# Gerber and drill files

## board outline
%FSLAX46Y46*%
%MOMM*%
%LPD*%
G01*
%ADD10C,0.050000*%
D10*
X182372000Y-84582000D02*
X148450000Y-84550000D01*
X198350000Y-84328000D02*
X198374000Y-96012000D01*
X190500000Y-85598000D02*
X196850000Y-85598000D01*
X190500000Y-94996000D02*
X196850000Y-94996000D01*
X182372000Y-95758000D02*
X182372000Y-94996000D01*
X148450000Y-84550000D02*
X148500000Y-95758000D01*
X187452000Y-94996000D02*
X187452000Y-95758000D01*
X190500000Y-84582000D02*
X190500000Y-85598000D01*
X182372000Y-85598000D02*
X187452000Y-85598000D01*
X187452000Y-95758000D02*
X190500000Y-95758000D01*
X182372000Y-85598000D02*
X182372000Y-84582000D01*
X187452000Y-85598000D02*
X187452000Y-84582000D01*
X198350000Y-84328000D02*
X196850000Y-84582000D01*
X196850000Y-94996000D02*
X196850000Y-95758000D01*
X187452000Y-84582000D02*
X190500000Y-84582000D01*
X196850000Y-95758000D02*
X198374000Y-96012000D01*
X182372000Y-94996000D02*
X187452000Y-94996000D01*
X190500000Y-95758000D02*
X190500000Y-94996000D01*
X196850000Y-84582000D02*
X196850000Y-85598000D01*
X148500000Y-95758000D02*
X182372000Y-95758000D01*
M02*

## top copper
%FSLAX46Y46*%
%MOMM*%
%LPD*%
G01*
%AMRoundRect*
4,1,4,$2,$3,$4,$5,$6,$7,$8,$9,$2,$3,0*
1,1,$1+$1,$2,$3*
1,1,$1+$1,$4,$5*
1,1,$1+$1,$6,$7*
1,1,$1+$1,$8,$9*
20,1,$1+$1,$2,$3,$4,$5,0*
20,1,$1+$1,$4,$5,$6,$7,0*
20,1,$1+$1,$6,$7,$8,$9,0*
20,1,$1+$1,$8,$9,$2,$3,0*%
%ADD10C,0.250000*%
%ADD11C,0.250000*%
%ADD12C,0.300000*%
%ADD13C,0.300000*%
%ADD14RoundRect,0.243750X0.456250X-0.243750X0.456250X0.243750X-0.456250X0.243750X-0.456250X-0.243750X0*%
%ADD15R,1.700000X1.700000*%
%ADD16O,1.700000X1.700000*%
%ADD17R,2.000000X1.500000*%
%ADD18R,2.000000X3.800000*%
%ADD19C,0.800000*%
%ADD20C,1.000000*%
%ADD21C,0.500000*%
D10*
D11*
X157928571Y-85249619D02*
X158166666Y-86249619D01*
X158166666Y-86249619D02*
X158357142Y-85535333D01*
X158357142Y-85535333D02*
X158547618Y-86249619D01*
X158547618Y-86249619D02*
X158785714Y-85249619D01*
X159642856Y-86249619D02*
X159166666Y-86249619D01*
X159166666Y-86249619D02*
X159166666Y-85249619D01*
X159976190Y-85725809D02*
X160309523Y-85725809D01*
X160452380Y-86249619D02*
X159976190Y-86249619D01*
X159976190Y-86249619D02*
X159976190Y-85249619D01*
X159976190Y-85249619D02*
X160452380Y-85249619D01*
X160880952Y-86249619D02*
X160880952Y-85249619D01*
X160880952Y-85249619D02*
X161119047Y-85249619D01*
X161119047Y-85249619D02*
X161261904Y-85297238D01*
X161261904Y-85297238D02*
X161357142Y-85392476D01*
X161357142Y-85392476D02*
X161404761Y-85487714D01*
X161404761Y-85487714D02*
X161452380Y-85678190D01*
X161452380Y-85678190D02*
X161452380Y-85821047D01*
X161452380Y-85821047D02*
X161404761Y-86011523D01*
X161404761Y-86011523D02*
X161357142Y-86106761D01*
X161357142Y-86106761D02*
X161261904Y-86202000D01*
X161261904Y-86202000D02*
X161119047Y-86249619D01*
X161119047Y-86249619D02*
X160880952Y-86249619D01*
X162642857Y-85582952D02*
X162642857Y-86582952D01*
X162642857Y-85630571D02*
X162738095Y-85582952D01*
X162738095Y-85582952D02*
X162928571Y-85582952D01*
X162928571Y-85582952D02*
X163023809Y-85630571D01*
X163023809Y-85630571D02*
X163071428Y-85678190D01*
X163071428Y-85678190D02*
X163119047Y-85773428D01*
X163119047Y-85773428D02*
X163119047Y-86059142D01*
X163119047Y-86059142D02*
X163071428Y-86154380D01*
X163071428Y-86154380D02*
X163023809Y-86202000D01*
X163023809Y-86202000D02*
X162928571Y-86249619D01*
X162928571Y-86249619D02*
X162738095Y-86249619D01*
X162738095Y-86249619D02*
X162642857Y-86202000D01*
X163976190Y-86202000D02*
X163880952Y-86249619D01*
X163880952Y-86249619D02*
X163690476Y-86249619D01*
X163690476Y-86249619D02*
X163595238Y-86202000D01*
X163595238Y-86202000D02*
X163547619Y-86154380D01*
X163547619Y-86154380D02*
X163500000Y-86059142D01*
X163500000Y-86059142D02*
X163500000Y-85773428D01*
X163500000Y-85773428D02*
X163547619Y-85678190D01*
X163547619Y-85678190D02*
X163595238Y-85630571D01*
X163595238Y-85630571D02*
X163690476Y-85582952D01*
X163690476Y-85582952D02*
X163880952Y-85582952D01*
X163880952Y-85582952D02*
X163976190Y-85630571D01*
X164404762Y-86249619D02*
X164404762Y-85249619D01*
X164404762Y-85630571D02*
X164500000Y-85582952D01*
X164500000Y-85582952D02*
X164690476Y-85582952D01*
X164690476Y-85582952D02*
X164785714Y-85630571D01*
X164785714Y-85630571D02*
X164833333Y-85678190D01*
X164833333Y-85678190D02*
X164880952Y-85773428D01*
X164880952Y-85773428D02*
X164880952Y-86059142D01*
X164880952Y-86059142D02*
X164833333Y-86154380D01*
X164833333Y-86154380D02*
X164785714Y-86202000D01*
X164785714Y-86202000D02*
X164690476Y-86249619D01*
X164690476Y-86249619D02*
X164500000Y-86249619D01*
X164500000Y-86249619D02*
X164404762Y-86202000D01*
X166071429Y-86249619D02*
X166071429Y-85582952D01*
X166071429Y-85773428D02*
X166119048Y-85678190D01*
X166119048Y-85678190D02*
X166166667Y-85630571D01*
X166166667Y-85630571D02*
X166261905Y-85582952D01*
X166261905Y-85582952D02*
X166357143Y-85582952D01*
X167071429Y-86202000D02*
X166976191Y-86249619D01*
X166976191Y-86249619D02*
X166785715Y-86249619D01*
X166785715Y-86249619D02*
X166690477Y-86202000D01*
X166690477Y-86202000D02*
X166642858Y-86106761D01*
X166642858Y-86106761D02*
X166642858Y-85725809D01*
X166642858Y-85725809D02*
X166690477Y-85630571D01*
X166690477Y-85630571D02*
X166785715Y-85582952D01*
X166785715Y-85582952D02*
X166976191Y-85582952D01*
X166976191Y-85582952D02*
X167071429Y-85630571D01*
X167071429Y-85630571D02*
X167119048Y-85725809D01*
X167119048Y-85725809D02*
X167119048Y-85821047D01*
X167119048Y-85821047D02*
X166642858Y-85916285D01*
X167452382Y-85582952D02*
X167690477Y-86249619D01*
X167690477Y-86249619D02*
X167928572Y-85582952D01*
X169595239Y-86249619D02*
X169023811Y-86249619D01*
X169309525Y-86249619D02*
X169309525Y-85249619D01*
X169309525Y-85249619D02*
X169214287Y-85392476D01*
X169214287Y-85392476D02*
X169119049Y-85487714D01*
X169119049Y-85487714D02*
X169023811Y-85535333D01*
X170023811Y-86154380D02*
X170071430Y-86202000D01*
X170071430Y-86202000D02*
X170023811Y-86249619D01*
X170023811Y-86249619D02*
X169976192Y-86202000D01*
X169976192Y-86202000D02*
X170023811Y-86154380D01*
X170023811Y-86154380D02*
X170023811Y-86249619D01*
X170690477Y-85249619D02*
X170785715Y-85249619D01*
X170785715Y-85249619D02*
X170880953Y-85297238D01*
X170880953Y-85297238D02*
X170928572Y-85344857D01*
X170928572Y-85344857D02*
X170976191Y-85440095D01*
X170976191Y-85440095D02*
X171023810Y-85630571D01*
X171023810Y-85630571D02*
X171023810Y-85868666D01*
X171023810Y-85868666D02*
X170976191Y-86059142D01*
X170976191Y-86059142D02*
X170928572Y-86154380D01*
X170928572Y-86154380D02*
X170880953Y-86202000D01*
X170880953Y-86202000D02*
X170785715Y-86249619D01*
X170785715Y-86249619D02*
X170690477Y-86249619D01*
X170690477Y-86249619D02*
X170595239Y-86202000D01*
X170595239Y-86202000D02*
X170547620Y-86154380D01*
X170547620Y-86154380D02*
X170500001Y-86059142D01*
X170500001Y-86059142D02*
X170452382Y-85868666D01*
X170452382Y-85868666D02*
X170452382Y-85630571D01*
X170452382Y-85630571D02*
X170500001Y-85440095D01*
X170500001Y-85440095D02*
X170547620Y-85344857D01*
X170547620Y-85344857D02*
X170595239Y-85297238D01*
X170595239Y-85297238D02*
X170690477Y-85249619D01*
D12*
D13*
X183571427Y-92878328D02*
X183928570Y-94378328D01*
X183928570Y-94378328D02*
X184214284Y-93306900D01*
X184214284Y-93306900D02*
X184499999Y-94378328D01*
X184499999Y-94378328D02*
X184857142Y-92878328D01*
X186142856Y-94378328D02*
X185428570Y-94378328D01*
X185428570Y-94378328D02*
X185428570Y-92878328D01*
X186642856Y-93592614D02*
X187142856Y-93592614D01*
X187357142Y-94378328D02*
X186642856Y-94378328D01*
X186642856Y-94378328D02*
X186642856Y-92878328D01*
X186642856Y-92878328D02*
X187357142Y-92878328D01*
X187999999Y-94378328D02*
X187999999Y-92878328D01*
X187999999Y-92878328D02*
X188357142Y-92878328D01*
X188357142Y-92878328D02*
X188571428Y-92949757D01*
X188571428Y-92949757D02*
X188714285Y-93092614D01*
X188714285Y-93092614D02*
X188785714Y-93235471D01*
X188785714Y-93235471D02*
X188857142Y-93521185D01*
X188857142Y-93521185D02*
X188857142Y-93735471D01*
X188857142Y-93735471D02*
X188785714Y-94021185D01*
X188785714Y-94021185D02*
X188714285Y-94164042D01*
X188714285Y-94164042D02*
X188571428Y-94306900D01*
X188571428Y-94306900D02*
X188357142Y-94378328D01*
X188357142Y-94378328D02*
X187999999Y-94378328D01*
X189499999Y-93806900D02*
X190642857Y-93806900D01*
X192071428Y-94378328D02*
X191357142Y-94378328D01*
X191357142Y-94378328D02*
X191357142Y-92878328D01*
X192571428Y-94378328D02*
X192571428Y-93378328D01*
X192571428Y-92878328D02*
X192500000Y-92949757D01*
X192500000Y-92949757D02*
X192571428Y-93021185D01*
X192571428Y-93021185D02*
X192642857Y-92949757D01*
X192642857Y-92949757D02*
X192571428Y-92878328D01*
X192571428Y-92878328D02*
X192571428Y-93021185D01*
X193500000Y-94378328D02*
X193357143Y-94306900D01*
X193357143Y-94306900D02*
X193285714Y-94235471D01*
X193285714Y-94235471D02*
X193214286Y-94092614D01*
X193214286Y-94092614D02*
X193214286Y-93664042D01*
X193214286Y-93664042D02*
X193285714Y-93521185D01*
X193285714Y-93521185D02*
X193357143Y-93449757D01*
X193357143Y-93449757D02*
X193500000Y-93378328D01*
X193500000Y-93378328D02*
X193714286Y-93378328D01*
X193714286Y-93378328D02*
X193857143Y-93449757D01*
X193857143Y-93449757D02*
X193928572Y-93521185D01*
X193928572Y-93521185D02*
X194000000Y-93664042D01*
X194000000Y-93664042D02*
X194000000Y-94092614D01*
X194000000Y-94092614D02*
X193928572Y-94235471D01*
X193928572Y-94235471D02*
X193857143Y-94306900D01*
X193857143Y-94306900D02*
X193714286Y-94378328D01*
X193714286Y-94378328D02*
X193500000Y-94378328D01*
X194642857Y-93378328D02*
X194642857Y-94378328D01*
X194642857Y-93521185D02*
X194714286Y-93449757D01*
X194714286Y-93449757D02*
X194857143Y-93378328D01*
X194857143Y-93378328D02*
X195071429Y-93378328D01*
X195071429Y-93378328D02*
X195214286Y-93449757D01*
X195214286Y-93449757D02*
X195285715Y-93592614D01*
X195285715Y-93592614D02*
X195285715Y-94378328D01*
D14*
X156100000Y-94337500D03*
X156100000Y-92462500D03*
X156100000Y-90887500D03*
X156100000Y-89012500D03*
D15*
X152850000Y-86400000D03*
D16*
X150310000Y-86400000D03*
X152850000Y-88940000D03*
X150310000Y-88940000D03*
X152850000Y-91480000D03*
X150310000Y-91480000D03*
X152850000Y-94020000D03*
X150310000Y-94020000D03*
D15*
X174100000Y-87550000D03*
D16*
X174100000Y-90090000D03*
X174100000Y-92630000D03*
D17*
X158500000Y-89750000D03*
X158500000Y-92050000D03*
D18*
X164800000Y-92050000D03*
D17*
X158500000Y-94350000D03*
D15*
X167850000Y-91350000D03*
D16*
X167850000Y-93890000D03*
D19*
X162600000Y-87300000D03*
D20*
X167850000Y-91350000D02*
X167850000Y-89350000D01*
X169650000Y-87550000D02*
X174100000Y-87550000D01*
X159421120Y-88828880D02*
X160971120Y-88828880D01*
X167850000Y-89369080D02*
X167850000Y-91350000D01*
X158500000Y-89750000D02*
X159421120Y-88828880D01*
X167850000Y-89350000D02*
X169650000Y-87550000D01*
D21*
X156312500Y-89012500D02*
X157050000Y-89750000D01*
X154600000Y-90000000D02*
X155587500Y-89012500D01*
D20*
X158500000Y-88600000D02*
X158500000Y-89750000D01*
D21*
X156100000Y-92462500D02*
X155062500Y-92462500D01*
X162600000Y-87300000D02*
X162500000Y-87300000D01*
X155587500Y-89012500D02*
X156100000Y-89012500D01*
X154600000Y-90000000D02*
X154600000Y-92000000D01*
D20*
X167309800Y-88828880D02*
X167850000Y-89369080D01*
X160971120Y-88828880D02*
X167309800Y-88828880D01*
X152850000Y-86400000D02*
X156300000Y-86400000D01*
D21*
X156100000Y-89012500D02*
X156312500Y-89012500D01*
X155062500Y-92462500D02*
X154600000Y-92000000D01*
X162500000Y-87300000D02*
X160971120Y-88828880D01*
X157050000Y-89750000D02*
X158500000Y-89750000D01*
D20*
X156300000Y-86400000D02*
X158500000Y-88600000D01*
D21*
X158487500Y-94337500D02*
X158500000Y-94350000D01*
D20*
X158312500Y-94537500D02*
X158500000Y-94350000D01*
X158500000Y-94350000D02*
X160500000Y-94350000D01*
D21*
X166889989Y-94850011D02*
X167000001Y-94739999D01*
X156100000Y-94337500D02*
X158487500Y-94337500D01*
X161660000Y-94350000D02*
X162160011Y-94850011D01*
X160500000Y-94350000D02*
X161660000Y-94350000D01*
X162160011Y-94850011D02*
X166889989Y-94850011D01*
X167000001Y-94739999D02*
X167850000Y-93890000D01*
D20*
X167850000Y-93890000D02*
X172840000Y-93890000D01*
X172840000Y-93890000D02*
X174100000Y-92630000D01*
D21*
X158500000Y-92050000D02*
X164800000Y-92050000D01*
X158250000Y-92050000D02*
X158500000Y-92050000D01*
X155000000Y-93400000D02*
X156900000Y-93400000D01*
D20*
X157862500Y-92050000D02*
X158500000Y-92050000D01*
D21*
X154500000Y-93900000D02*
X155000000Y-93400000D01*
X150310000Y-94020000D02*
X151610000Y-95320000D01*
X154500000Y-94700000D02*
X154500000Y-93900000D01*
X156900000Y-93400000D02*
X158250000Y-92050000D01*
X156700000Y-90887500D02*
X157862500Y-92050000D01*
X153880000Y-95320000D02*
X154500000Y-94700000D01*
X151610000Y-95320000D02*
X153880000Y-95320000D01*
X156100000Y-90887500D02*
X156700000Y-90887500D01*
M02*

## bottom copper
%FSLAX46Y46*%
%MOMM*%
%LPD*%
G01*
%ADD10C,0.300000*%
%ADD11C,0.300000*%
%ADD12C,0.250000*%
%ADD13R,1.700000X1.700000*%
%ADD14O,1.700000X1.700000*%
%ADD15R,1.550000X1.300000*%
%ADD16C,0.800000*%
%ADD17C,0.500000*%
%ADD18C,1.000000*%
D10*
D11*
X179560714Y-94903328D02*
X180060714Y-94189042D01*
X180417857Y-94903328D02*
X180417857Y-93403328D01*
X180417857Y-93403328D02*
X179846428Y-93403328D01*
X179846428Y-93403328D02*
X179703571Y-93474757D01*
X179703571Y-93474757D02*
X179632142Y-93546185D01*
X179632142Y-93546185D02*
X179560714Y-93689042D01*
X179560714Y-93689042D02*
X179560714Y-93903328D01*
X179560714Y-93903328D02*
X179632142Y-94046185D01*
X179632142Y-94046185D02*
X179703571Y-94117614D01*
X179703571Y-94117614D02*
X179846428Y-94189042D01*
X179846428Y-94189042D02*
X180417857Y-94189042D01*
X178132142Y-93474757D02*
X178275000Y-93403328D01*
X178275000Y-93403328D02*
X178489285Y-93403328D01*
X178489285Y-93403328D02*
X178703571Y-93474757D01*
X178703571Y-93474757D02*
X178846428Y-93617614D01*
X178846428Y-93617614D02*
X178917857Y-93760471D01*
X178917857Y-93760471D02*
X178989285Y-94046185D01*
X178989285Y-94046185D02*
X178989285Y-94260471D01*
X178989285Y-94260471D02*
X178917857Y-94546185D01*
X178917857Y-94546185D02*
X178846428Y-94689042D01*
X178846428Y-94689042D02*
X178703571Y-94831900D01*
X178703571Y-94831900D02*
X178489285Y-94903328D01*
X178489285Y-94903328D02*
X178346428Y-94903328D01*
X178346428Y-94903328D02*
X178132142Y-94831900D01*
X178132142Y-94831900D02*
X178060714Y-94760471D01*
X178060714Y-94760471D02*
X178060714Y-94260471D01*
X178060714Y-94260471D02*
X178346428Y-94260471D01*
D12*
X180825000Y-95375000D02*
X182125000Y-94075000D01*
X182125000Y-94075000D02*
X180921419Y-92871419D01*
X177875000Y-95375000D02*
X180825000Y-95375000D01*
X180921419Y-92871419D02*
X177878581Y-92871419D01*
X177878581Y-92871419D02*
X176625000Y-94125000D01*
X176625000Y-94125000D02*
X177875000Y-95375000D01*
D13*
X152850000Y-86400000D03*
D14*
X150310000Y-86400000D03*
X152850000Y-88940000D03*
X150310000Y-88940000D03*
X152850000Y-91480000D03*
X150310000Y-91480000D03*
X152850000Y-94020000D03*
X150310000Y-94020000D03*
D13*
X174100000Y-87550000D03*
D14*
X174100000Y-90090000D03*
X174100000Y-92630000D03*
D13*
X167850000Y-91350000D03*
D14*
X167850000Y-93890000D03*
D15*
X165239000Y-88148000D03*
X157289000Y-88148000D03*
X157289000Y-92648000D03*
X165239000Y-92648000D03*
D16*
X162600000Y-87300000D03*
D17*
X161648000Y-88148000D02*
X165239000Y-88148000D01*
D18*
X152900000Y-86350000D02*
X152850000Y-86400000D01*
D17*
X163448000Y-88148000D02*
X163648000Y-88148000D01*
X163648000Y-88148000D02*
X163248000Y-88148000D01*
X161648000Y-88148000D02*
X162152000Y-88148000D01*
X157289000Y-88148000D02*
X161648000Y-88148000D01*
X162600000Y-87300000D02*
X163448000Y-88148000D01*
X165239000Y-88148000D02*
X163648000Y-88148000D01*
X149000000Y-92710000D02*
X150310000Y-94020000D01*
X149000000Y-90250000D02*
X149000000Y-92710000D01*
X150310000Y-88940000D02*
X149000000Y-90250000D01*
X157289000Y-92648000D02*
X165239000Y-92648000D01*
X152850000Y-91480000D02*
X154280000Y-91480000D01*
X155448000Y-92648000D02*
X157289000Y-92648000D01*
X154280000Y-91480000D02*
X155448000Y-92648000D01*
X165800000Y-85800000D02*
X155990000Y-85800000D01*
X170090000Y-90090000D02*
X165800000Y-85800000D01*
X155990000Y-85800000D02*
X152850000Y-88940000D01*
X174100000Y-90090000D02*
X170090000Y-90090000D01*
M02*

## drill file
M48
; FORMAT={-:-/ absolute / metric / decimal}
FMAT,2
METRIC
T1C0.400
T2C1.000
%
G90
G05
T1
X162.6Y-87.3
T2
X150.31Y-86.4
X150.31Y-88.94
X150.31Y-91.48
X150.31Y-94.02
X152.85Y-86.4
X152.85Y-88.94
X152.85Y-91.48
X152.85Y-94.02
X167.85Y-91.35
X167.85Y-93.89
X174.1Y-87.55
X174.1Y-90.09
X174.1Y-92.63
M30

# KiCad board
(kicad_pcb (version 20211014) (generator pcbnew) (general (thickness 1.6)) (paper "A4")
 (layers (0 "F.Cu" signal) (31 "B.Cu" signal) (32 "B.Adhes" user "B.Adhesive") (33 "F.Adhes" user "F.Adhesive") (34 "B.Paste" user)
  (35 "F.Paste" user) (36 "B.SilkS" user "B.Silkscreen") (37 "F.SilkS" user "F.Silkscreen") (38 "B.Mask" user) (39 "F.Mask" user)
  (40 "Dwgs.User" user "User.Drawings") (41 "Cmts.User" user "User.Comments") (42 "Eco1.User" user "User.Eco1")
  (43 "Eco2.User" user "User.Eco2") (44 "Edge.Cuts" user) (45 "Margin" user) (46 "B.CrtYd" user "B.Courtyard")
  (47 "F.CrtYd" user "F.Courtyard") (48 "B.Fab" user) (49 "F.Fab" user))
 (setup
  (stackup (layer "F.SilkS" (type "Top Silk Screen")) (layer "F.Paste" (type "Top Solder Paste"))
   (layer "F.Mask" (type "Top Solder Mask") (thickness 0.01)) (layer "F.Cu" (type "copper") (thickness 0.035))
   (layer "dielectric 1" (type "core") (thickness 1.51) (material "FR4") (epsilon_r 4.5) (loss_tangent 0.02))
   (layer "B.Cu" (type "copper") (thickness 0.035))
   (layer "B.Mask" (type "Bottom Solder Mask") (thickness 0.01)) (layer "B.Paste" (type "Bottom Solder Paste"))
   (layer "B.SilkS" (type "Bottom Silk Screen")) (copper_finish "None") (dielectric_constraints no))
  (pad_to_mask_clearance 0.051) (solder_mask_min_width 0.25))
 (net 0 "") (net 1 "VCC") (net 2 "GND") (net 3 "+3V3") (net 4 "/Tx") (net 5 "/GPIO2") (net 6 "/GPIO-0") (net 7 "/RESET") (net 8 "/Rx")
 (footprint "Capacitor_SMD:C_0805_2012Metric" (layer "F.Cu") (at 156.1 93.4 90)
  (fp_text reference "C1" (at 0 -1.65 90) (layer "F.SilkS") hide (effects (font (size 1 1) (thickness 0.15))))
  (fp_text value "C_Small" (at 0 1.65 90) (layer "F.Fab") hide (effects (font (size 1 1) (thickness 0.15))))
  (pad "1" smd roundrect locked (at -0.9375 0 90) (size 0.975 1.4) (layers "F.Cu" "F.Paste" "F.Mask") (roundrect_rratio 0.25) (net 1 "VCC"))
  (pad "2" smd roundrect locked (at 0.9375 0 90) (size 0.975 1.4) (layers "F.Cu" "F.Paste" "F.Mask") (roundrect_rratio 0.25) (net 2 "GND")))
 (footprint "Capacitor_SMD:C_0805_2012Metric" (layer "F.Cu") (at 156.1 89.95 90)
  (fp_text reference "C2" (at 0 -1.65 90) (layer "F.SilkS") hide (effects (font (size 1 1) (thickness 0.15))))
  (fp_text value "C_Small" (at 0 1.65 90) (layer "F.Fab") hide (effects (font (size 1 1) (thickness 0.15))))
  (pad "1" smd roundrect locked (at -0.9375 0 90) (size 0.975 1.4) (layers "F.Cu" "F.Paste" "F.Mask") (roundrect_rratio 0.25) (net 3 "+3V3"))
  (pad "2" smd roundrect locked (at 0.9375 0 90) (size 0.975 1.4) (layers "F.Cu" "F.Paste" "F.Mask") (roundrect_rratio 0.25) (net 2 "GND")))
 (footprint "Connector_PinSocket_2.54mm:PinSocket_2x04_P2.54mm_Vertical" (layer "F.Cu") (at 152.85 86.4)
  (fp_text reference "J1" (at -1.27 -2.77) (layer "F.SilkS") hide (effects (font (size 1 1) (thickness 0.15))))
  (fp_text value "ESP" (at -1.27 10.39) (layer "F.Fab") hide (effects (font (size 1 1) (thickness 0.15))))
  (pad "1" thru_hole rect locked (at 0 0) (size 1.7 1.7) (drill 1) (layers *.Cu *.Mask) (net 2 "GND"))
  (pad "2" thru_hole oval locked (at -2.54 0) (size 1.7 1.7) (drill 1) (layers *.Cu *.Mask) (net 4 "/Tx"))
  (pad "3" thru_hole oval locked (at 0 2.54) (size 1.7 1.7) (drill 1) (layers *.Cu *.Mask) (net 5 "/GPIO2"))
  (pad "4" thru_hole oval locked (at -2.54 2.54) (size 1.7 1.7) (drill 1) (layers *.Cu *.Mask) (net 3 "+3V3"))
  (pad "5" thru_hole oval locked (at 0 5.08) (size 1.7 1.7) (drill 1) (layers *.Cu *.Mask) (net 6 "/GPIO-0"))
  (pad "6" thru_hole oval locked (at -2.54 5.08) (size 1.7 1.7) (drill 1) (layers *.Cu *.Mask) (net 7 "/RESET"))
  (pad "7" thru_hole oval locked (at 0 7.62) (size 1.7 1.7) (drill 1) (layers *.Cu *.Mask) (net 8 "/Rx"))
  (pad "8" thru_hole oval locked (at -2.54 7.62) (size 1.7 1.7) (drill 1) (layers *.Cu *.Mask) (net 3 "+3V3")))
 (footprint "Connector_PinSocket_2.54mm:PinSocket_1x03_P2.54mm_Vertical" (layer "F.Cu") (at 174.1 87.55)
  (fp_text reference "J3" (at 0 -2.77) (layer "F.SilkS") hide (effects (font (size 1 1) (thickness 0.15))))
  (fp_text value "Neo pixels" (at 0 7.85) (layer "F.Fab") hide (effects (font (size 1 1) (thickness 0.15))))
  (pad "1" thru_hole rect locked (at 0 0) (size 1.7 1.7) (drill 1) (layers *.Cu *.Mask) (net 2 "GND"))
  (pad "2" thru_hole oval locked (at 0 2.54) (size 1.7 1.7) (drill 1) (layers *.Cu *.Mask) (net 5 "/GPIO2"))
  (pad "3" thru_hole oval locked (at 0 5.08) (size 1.7 1.7) (drill 1) (layers *.Cu *.Mask) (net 1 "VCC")))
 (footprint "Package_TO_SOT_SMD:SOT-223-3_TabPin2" (layer "F.Cu") (at 161.65 92.05)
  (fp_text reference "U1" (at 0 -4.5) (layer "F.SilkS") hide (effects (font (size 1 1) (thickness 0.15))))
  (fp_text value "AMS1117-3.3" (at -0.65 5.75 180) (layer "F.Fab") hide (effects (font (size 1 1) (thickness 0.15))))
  (pad "1" smd rect locked (at -3.15 -2.3) (size 2 1.5) (layers "F.Cu" "F.Paste" "F.Mask") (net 2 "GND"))
  (pad "2" smd rect locked (at -3.15 0) (size 2 1.5) (layers "F.Cu" "F.Paste" "F.Mask") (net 3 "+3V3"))
  (pad "2" smd rect locked (at 3.15 0) (size 2 3.8) (layers "F.Cu" "F.Paste" "F.Mask") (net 3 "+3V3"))
  (pad "3" smd rect locked (at -3.15 2.3) (size 2 1.5) (layers "F.Cu" "F.Paste" "F.Mask") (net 1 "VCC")))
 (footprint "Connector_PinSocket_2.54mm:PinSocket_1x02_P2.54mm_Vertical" (layer "F.Cu") (at 167.85 91.35)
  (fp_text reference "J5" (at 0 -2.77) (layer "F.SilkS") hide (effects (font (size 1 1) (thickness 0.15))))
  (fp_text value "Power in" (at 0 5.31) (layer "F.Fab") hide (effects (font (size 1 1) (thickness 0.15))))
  (pad "1" thru_hole rect locked (at 0 0) (size 1.7 1.7) (drill 1) (layers *.Cu *.Mask) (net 2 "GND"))
  (pad "2" thru_hole oval locked (at 0 2.54) (size 1.7 1.7) (drill 1) (layers *.Cu *.Mask) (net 1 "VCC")))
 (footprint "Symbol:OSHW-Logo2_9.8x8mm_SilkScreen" (layer "F.Cu") (at 189 89.1)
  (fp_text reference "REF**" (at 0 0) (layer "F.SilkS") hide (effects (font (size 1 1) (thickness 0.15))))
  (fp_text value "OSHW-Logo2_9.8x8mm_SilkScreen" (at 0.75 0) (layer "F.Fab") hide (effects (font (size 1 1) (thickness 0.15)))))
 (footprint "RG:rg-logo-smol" (layer "F.Cu") (at 179.3 94.1 180)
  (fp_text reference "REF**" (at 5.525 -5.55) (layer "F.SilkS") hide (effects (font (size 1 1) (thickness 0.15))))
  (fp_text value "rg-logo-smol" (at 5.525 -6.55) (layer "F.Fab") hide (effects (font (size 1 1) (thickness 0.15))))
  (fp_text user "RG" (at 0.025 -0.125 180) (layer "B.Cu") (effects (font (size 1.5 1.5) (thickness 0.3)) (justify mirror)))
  (fp_line (start -1.525 -1.275) (end -2.825 0.025) (layer "B.Cu") (width 0.25))
  (fp_line (start -2.825 0.025) (end -1.621419 1.228581) (layer "B.Cu") (width 0.25))
  (fp_line (start 1.425 -1.275) (end -1.525 -1.275) (layer "B.Cu") (width 0.25))
  (fp_line (start -1.621419 1.228581) (end 1.421419 1.228581) (layer "B.Cu") (width 0.25))
  (fp_line (start 1.421419 1.228581) (end 2.675 -0.025) (layer "B.Cu") (width 0.25))
  (fp_line (start 2.675 -0.025) (end 1.425 -1.275) (layer "B.Cu") (width 0.25)))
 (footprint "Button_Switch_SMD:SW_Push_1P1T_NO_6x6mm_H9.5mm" (layer "B.Cu") (at 161.264 90.398 180)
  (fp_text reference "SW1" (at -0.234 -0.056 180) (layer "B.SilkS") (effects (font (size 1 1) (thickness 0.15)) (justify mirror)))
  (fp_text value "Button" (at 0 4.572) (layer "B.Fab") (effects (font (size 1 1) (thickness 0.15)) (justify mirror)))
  (pad "1" smd rect locked (at -3.975 2.25 180) (size 1.55 1.3) (layers "B.Cu" "B.Paste" "B.Mask") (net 2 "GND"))
  (pad "1" smd rect locked (at 3.975 2.25 180) (size 1.55 1.3) (layers "B.Cu" "B.Paste" "B.Mask") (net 2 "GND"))
  (pad "2" smd rect locked (at 3.975 -2.25 180) (size 1.55 1.3) (layers "B.Cu" "B.Paste" "B.Mask") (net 6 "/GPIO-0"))
  (pad "2" smd rect locked (at -3.975 -2.25 180) (size 1.55 1.3) (layers "B.Cu" "B.Paste" "B.Mask") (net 6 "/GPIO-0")))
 (gr_line (start 182.372 84.582) (end 148.45 84.55) (layer "Edge.Cuts") (width 0.05))
 (gr_line (start 198.35 84.328) (end 198.374 96.012) (layer "Edge.Cuts") (width 0.05))
 (gr_line (start 190.5 85.598) (end 196.85 85.598) (layer "Edge.Cuts") (width 0.05))
 (gr_line (start 190.5 94.996) (end 196.85 94.996) (layer "Edge.Cuts") (width 0.05))
 (gr_line (start 182.372 95.758) (end 182.372 94.996) (layer "Edge.Cuts") (width 0.05))
 (gr_line (start 148.45 84.55) (end 148.5 95.758) (layer "Edge.Cuts") (width 0.05))
 (gr_line (start 187.452 94.996) (end 187.452 95.758) (layer "Edge.Cuts") (width 0.05))
 (gr_line (start 190.5 84.582) (end 190.5 85.598) (layer "Edge.Cuts") (width 0.05))
 (gr_line (start 182.372 85.598) (end 187.452 85.598) (layer "Edge.Cuts") (width 0.05))
 (gr_line (start 187.452 95.758) (end 190.5 95.758) (layer "Edge.Cuts") (width 0.05))
 (gr_line (start 182.372 85.598) (end 182.372 84.582) (layer "Edge.Cuts") (width 0.05))
 (gr_line (start 187.452 85.598) (end 187.452 84.582) (layer "Edge.Cuts") (width 0.05))
 (gr_line (start 198.35 84.328) (end 196.85 84.582) (layer "Edge.Cuts") (width 0.05))
 (gr_line (start 196.85 94.996) (end 196.85 95.758) (layer "Edge.Cuts") (width 0.05))
 (gr_line (start 187.452 84.582) (end 190.5 84.582) (layer "Edge.Cuts") (width 0.05))
 (gr_line (start 196.85 95.758) (end 198.374 96.012) (layer "Edge.Cuts") (width 0.05))
 (gr_line (start 182.372 94.996) (end 187.452 94.996) (layer "Edge.Cuts") (width 0.05))
 (gr_line (start 190.5 95.758) (end 190.5 94.996) (layer "Edge.Cuts") (width 0.05))
 (gr_line (start 196.85 84.582) (end 196.85 85.598) (layer "Edge.Cuts") (width 0.05))
 (gr_line (start 148.5 95.758) (end 182.372 95.758) (layer "Edge.Cuts") (width 0.05))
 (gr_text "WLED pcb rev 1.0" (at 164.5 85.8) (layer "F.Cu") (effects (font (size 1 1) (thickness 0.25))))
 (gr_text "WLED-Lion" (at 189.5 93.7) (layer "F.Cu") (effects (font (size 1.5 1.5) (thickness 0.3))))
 (segment (start 167.85 91.35) (end 167.85 89.35) (width 1) (layer "F.Cu") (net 2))
 (segment (start 169.65 87.55) (end 174.1 87.55) (width 1) (layer "F.Cu") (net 2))
 (segment (start 159.42112 88.82888) (end 160.97112 88.82888) (width 1) (layer "F.Cu") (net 2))
 (segment (start 167.85 89.36908) (end 167.85 91.35) (width 1) (layer "F.Cu") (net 2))
 (segment (start 158.5 89.75) (end 159.42112 88.82888) (width 1) (layer "F.Cu") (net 2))
 (segment (start 167.85 89.35) (end 169.65 87.55) (width 1) (layer "F.Cu") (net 2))
 (segment (start 156.3125 89.0125) (end 157.05 89.75) (width 0.5) (layer "F.Cu") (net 2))
 (segment (start 154.6 90) (end 155.5875 89.0125) (width 0.5) (layer "F.Cu") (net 2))
 (segment (start 158.5 88.6) (end 158.5 89.75) (width 1) (layer "F.Cu") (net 2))
 (segment (start 156.1 92.4625) (end 155.0625 92.4625) (width 0.5) (layer "F.Cu") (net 2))
 (segment (start 162.6 87.3) (end 162.5 87.3) (width 0.5) (layer "F.Cu") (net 2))
 (segment (start 155.5875 89.0125) (end 156.1 89.0125) (width 0.5) (layer "F.Cu") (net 2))
 (segment (start 154.6 90) (end 154.6 92) (width 0.5) (layer "F.Cu") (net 2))
 (segment (start 167.3098 88.82888) (end 167.85 89.36908) (width 1) (layer "F.Cu") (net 2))
 (segment (start 160.97112 88.82888) (end 167.3098 88.82888) (width 1) (layer "F.Cu") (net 2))
 (segment (start 152.85 86.4) (end 156.3 86.4) (width 1) (layer "F.Cu") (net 2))
 (segment (start 156.1 89.0125) (end 156.3125 89.0125) (width 0.5) (layer "F.Cu") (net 2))
 (segment (start 155.0625 92.4625) (end 154.6 92) (width 0.5) (layer "F.Cu") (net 2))
 (segment (start 162.5 87.3) (end 160.97112 88.82888) (width 0.5) (layer "F.Cu") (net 2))
 (segment (start 157.05 89.75) (end 158.5 89.75) (width 0.5) (layer "F.Cu") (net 2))
 (segment (start 156.3 86.4) (end 158.5 88.6) (width 1) (layer "F.Cu") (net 2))
 (via (at 162.6 87.3) (size 0.8) (drill 0.4) (layers "F.Cu" "B.Cu") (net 2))
 (segment (start 161.648 88.148) (end 165.239 88.148) (width 0.5) (layer "B.Cu") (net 2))
 (segment (start 152.9 86.35) (end 152.85 86.4) (width 1) (layer "B.Cu") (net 2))
 (segment (start 163.448 88.148) (end 163.648 88.148) (width 0.5) (layer "B.Cu") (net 2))
 (segment (start 163.648 88.148) (end 163.248 88.148) (width 0.5) (layer "B.Cu") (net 2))
 (segment (start 161.648 88.148) (end 162.152 88.148) (width 0.5) (layer "B.Cu") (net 2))
 (segment (start 157.289 88.148) (end 161.648 88.148) (width 0.5) (layer "B.Cu") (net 2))
 (segment (start 162.6 87.3) (end 163.448 88.148) (width 0.5) (layer "B.Cu") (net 2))
 (segment (start 165.239 88.148) (end 163.648 88.148) (width 0.5) (layer "B.Cu") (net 2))
 (segment (start 158.4875 94.3375) (end 158.5 94.35) (width 0.5) (layer "F.Cu") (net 1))
 (segment (start 158.3125 94.5375) (end 158.5 94.35) (width 1) (layer "F.Cu") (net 1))
 (segment (start 158.5 94.35) (end 160.5 94.35) (width 1) (layer "F.Cu") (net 1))
 (segment (start 166.889989 94.850011) (end 167.000001 94.739999) (width 0.5) (layer "F.Cu") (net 1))
 (segment (start 156.1 94.3375) (end 158.4875 94.3375) (width 0.5) (layer "F.Cu") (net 1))
 (segment (start 161.66 94.35) (end 162.160011 94.850011) (width 0.5) (layer "F.Cu") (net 1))
 (segment (start 160.5 94.35) (end 161.66 94.35) (width 0.5) (layer "F.Cu") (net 1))
 (segment (start 162.160011 94.850011) (end 166.889989 94.850011) (width 0.5) (layer "F.Cu") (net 1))
 (segment (start 167.000001 94.739999) (end 167.85 93.89) (width 0.5) (layer "F.Cu") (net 1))
 (segment (start 167.85 93.89) (end 172.84 93.89) (width 1) (layer "F.Cu") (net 1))
 (segment (start 172.84 93.89) (end 174.1 92.63) (width 1) (layer "F.Cu") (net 1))
 (segment (start 158.5 92.05) (end 164.8 92.05) (width 0.5) (layer "F.Cu") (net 3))
 (segment (start 158.25 92.05) (end 158.5 92.05) (width 0.5) (layer "F.Cu") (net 3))
 (segment (start 155 93.4) (end 156.9 93.4) (width 0.5) (layer "F.Cu") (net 3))
 (segment (start 157.8625 92.05) (end 158.5 92.05) (width 1) (layer "F.Cu") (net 3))
 (segment (start 154.5 93.9) (end 155 93.4) (width 0.5) (layer "F.Cu") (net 3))
 (segment (start 150.31 94.02) (end 151.61 95.32) (width 0.5) (layer "F.Cu") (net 3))
 (segment (start 154.5 94.7) (end 154.5 93.9) (width 0.5) (layer "F.Cu") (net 3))
 (segment (start 156.9 93.4) (end 158.25 92.05) (width 0.5) (layer "F.Cu") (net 3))
 (segment (start 156.7 90.8875) (end 157.8625 92.05) (width 0.5) (layer "F.Cu") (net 3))
 (segment (start 153.88 95.32) (end 154.5 94.7) (width 0.5) (layer "F.Cu") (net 3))
 (segment (start 151.61 95.32) (end 153.88 95.32) (width 0.5) (layer "F.Cu") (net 3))
 (segment (start 156.1 90.8875) (end 156.7 90.8875) (width 0.5) (layer "F.Cu") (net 3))
 (segment (start 149 92.71) (end 150.31 94.02) (width 0.5) (layer "B.Cu") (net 3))
 (segment (start 149 90.25) (end 149 92.71) (width 0.5) (layer "B.Cu") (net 3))
 (segment (start 150.31 88.94) (end 149 90.25) (width 0.5) (layer "B.Cu") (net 3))
 (segment (start 157.289 92.648) (end 165.239 92.648) (width 0.5) (layer "B.Cu") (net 6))
 (segment (start 152.85 91.48) (end 154.28 91.48) (width 0.5) (layer "B.Cu") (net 6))
 (segment (start 155.448 92.648) (end 157.289 92.648) (width 0.5) (layer "B.Cu") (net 6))
 (segment (start 154.28 91.48) (end 155.448 92.648) (width 0.5) (layer "B.Cu") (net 6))
 (segment (start 165.8 85.8) (end 155.99 85.8) (width 0.5) (layer "B.Cu") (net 5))
 (segment (start 170.09 90.09) (end 165.8 85.8) (width 0.5) (layer "B.Cu") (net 5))
 (segment (start 155.99 85.8) (end 152.85 88.94) (width 0.5) (layer "B.Cu") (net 5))
 (segment (start 174.1 90.09) (end 170.09 90.09) (width 0.5) (layer "B.Cu") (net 5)))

